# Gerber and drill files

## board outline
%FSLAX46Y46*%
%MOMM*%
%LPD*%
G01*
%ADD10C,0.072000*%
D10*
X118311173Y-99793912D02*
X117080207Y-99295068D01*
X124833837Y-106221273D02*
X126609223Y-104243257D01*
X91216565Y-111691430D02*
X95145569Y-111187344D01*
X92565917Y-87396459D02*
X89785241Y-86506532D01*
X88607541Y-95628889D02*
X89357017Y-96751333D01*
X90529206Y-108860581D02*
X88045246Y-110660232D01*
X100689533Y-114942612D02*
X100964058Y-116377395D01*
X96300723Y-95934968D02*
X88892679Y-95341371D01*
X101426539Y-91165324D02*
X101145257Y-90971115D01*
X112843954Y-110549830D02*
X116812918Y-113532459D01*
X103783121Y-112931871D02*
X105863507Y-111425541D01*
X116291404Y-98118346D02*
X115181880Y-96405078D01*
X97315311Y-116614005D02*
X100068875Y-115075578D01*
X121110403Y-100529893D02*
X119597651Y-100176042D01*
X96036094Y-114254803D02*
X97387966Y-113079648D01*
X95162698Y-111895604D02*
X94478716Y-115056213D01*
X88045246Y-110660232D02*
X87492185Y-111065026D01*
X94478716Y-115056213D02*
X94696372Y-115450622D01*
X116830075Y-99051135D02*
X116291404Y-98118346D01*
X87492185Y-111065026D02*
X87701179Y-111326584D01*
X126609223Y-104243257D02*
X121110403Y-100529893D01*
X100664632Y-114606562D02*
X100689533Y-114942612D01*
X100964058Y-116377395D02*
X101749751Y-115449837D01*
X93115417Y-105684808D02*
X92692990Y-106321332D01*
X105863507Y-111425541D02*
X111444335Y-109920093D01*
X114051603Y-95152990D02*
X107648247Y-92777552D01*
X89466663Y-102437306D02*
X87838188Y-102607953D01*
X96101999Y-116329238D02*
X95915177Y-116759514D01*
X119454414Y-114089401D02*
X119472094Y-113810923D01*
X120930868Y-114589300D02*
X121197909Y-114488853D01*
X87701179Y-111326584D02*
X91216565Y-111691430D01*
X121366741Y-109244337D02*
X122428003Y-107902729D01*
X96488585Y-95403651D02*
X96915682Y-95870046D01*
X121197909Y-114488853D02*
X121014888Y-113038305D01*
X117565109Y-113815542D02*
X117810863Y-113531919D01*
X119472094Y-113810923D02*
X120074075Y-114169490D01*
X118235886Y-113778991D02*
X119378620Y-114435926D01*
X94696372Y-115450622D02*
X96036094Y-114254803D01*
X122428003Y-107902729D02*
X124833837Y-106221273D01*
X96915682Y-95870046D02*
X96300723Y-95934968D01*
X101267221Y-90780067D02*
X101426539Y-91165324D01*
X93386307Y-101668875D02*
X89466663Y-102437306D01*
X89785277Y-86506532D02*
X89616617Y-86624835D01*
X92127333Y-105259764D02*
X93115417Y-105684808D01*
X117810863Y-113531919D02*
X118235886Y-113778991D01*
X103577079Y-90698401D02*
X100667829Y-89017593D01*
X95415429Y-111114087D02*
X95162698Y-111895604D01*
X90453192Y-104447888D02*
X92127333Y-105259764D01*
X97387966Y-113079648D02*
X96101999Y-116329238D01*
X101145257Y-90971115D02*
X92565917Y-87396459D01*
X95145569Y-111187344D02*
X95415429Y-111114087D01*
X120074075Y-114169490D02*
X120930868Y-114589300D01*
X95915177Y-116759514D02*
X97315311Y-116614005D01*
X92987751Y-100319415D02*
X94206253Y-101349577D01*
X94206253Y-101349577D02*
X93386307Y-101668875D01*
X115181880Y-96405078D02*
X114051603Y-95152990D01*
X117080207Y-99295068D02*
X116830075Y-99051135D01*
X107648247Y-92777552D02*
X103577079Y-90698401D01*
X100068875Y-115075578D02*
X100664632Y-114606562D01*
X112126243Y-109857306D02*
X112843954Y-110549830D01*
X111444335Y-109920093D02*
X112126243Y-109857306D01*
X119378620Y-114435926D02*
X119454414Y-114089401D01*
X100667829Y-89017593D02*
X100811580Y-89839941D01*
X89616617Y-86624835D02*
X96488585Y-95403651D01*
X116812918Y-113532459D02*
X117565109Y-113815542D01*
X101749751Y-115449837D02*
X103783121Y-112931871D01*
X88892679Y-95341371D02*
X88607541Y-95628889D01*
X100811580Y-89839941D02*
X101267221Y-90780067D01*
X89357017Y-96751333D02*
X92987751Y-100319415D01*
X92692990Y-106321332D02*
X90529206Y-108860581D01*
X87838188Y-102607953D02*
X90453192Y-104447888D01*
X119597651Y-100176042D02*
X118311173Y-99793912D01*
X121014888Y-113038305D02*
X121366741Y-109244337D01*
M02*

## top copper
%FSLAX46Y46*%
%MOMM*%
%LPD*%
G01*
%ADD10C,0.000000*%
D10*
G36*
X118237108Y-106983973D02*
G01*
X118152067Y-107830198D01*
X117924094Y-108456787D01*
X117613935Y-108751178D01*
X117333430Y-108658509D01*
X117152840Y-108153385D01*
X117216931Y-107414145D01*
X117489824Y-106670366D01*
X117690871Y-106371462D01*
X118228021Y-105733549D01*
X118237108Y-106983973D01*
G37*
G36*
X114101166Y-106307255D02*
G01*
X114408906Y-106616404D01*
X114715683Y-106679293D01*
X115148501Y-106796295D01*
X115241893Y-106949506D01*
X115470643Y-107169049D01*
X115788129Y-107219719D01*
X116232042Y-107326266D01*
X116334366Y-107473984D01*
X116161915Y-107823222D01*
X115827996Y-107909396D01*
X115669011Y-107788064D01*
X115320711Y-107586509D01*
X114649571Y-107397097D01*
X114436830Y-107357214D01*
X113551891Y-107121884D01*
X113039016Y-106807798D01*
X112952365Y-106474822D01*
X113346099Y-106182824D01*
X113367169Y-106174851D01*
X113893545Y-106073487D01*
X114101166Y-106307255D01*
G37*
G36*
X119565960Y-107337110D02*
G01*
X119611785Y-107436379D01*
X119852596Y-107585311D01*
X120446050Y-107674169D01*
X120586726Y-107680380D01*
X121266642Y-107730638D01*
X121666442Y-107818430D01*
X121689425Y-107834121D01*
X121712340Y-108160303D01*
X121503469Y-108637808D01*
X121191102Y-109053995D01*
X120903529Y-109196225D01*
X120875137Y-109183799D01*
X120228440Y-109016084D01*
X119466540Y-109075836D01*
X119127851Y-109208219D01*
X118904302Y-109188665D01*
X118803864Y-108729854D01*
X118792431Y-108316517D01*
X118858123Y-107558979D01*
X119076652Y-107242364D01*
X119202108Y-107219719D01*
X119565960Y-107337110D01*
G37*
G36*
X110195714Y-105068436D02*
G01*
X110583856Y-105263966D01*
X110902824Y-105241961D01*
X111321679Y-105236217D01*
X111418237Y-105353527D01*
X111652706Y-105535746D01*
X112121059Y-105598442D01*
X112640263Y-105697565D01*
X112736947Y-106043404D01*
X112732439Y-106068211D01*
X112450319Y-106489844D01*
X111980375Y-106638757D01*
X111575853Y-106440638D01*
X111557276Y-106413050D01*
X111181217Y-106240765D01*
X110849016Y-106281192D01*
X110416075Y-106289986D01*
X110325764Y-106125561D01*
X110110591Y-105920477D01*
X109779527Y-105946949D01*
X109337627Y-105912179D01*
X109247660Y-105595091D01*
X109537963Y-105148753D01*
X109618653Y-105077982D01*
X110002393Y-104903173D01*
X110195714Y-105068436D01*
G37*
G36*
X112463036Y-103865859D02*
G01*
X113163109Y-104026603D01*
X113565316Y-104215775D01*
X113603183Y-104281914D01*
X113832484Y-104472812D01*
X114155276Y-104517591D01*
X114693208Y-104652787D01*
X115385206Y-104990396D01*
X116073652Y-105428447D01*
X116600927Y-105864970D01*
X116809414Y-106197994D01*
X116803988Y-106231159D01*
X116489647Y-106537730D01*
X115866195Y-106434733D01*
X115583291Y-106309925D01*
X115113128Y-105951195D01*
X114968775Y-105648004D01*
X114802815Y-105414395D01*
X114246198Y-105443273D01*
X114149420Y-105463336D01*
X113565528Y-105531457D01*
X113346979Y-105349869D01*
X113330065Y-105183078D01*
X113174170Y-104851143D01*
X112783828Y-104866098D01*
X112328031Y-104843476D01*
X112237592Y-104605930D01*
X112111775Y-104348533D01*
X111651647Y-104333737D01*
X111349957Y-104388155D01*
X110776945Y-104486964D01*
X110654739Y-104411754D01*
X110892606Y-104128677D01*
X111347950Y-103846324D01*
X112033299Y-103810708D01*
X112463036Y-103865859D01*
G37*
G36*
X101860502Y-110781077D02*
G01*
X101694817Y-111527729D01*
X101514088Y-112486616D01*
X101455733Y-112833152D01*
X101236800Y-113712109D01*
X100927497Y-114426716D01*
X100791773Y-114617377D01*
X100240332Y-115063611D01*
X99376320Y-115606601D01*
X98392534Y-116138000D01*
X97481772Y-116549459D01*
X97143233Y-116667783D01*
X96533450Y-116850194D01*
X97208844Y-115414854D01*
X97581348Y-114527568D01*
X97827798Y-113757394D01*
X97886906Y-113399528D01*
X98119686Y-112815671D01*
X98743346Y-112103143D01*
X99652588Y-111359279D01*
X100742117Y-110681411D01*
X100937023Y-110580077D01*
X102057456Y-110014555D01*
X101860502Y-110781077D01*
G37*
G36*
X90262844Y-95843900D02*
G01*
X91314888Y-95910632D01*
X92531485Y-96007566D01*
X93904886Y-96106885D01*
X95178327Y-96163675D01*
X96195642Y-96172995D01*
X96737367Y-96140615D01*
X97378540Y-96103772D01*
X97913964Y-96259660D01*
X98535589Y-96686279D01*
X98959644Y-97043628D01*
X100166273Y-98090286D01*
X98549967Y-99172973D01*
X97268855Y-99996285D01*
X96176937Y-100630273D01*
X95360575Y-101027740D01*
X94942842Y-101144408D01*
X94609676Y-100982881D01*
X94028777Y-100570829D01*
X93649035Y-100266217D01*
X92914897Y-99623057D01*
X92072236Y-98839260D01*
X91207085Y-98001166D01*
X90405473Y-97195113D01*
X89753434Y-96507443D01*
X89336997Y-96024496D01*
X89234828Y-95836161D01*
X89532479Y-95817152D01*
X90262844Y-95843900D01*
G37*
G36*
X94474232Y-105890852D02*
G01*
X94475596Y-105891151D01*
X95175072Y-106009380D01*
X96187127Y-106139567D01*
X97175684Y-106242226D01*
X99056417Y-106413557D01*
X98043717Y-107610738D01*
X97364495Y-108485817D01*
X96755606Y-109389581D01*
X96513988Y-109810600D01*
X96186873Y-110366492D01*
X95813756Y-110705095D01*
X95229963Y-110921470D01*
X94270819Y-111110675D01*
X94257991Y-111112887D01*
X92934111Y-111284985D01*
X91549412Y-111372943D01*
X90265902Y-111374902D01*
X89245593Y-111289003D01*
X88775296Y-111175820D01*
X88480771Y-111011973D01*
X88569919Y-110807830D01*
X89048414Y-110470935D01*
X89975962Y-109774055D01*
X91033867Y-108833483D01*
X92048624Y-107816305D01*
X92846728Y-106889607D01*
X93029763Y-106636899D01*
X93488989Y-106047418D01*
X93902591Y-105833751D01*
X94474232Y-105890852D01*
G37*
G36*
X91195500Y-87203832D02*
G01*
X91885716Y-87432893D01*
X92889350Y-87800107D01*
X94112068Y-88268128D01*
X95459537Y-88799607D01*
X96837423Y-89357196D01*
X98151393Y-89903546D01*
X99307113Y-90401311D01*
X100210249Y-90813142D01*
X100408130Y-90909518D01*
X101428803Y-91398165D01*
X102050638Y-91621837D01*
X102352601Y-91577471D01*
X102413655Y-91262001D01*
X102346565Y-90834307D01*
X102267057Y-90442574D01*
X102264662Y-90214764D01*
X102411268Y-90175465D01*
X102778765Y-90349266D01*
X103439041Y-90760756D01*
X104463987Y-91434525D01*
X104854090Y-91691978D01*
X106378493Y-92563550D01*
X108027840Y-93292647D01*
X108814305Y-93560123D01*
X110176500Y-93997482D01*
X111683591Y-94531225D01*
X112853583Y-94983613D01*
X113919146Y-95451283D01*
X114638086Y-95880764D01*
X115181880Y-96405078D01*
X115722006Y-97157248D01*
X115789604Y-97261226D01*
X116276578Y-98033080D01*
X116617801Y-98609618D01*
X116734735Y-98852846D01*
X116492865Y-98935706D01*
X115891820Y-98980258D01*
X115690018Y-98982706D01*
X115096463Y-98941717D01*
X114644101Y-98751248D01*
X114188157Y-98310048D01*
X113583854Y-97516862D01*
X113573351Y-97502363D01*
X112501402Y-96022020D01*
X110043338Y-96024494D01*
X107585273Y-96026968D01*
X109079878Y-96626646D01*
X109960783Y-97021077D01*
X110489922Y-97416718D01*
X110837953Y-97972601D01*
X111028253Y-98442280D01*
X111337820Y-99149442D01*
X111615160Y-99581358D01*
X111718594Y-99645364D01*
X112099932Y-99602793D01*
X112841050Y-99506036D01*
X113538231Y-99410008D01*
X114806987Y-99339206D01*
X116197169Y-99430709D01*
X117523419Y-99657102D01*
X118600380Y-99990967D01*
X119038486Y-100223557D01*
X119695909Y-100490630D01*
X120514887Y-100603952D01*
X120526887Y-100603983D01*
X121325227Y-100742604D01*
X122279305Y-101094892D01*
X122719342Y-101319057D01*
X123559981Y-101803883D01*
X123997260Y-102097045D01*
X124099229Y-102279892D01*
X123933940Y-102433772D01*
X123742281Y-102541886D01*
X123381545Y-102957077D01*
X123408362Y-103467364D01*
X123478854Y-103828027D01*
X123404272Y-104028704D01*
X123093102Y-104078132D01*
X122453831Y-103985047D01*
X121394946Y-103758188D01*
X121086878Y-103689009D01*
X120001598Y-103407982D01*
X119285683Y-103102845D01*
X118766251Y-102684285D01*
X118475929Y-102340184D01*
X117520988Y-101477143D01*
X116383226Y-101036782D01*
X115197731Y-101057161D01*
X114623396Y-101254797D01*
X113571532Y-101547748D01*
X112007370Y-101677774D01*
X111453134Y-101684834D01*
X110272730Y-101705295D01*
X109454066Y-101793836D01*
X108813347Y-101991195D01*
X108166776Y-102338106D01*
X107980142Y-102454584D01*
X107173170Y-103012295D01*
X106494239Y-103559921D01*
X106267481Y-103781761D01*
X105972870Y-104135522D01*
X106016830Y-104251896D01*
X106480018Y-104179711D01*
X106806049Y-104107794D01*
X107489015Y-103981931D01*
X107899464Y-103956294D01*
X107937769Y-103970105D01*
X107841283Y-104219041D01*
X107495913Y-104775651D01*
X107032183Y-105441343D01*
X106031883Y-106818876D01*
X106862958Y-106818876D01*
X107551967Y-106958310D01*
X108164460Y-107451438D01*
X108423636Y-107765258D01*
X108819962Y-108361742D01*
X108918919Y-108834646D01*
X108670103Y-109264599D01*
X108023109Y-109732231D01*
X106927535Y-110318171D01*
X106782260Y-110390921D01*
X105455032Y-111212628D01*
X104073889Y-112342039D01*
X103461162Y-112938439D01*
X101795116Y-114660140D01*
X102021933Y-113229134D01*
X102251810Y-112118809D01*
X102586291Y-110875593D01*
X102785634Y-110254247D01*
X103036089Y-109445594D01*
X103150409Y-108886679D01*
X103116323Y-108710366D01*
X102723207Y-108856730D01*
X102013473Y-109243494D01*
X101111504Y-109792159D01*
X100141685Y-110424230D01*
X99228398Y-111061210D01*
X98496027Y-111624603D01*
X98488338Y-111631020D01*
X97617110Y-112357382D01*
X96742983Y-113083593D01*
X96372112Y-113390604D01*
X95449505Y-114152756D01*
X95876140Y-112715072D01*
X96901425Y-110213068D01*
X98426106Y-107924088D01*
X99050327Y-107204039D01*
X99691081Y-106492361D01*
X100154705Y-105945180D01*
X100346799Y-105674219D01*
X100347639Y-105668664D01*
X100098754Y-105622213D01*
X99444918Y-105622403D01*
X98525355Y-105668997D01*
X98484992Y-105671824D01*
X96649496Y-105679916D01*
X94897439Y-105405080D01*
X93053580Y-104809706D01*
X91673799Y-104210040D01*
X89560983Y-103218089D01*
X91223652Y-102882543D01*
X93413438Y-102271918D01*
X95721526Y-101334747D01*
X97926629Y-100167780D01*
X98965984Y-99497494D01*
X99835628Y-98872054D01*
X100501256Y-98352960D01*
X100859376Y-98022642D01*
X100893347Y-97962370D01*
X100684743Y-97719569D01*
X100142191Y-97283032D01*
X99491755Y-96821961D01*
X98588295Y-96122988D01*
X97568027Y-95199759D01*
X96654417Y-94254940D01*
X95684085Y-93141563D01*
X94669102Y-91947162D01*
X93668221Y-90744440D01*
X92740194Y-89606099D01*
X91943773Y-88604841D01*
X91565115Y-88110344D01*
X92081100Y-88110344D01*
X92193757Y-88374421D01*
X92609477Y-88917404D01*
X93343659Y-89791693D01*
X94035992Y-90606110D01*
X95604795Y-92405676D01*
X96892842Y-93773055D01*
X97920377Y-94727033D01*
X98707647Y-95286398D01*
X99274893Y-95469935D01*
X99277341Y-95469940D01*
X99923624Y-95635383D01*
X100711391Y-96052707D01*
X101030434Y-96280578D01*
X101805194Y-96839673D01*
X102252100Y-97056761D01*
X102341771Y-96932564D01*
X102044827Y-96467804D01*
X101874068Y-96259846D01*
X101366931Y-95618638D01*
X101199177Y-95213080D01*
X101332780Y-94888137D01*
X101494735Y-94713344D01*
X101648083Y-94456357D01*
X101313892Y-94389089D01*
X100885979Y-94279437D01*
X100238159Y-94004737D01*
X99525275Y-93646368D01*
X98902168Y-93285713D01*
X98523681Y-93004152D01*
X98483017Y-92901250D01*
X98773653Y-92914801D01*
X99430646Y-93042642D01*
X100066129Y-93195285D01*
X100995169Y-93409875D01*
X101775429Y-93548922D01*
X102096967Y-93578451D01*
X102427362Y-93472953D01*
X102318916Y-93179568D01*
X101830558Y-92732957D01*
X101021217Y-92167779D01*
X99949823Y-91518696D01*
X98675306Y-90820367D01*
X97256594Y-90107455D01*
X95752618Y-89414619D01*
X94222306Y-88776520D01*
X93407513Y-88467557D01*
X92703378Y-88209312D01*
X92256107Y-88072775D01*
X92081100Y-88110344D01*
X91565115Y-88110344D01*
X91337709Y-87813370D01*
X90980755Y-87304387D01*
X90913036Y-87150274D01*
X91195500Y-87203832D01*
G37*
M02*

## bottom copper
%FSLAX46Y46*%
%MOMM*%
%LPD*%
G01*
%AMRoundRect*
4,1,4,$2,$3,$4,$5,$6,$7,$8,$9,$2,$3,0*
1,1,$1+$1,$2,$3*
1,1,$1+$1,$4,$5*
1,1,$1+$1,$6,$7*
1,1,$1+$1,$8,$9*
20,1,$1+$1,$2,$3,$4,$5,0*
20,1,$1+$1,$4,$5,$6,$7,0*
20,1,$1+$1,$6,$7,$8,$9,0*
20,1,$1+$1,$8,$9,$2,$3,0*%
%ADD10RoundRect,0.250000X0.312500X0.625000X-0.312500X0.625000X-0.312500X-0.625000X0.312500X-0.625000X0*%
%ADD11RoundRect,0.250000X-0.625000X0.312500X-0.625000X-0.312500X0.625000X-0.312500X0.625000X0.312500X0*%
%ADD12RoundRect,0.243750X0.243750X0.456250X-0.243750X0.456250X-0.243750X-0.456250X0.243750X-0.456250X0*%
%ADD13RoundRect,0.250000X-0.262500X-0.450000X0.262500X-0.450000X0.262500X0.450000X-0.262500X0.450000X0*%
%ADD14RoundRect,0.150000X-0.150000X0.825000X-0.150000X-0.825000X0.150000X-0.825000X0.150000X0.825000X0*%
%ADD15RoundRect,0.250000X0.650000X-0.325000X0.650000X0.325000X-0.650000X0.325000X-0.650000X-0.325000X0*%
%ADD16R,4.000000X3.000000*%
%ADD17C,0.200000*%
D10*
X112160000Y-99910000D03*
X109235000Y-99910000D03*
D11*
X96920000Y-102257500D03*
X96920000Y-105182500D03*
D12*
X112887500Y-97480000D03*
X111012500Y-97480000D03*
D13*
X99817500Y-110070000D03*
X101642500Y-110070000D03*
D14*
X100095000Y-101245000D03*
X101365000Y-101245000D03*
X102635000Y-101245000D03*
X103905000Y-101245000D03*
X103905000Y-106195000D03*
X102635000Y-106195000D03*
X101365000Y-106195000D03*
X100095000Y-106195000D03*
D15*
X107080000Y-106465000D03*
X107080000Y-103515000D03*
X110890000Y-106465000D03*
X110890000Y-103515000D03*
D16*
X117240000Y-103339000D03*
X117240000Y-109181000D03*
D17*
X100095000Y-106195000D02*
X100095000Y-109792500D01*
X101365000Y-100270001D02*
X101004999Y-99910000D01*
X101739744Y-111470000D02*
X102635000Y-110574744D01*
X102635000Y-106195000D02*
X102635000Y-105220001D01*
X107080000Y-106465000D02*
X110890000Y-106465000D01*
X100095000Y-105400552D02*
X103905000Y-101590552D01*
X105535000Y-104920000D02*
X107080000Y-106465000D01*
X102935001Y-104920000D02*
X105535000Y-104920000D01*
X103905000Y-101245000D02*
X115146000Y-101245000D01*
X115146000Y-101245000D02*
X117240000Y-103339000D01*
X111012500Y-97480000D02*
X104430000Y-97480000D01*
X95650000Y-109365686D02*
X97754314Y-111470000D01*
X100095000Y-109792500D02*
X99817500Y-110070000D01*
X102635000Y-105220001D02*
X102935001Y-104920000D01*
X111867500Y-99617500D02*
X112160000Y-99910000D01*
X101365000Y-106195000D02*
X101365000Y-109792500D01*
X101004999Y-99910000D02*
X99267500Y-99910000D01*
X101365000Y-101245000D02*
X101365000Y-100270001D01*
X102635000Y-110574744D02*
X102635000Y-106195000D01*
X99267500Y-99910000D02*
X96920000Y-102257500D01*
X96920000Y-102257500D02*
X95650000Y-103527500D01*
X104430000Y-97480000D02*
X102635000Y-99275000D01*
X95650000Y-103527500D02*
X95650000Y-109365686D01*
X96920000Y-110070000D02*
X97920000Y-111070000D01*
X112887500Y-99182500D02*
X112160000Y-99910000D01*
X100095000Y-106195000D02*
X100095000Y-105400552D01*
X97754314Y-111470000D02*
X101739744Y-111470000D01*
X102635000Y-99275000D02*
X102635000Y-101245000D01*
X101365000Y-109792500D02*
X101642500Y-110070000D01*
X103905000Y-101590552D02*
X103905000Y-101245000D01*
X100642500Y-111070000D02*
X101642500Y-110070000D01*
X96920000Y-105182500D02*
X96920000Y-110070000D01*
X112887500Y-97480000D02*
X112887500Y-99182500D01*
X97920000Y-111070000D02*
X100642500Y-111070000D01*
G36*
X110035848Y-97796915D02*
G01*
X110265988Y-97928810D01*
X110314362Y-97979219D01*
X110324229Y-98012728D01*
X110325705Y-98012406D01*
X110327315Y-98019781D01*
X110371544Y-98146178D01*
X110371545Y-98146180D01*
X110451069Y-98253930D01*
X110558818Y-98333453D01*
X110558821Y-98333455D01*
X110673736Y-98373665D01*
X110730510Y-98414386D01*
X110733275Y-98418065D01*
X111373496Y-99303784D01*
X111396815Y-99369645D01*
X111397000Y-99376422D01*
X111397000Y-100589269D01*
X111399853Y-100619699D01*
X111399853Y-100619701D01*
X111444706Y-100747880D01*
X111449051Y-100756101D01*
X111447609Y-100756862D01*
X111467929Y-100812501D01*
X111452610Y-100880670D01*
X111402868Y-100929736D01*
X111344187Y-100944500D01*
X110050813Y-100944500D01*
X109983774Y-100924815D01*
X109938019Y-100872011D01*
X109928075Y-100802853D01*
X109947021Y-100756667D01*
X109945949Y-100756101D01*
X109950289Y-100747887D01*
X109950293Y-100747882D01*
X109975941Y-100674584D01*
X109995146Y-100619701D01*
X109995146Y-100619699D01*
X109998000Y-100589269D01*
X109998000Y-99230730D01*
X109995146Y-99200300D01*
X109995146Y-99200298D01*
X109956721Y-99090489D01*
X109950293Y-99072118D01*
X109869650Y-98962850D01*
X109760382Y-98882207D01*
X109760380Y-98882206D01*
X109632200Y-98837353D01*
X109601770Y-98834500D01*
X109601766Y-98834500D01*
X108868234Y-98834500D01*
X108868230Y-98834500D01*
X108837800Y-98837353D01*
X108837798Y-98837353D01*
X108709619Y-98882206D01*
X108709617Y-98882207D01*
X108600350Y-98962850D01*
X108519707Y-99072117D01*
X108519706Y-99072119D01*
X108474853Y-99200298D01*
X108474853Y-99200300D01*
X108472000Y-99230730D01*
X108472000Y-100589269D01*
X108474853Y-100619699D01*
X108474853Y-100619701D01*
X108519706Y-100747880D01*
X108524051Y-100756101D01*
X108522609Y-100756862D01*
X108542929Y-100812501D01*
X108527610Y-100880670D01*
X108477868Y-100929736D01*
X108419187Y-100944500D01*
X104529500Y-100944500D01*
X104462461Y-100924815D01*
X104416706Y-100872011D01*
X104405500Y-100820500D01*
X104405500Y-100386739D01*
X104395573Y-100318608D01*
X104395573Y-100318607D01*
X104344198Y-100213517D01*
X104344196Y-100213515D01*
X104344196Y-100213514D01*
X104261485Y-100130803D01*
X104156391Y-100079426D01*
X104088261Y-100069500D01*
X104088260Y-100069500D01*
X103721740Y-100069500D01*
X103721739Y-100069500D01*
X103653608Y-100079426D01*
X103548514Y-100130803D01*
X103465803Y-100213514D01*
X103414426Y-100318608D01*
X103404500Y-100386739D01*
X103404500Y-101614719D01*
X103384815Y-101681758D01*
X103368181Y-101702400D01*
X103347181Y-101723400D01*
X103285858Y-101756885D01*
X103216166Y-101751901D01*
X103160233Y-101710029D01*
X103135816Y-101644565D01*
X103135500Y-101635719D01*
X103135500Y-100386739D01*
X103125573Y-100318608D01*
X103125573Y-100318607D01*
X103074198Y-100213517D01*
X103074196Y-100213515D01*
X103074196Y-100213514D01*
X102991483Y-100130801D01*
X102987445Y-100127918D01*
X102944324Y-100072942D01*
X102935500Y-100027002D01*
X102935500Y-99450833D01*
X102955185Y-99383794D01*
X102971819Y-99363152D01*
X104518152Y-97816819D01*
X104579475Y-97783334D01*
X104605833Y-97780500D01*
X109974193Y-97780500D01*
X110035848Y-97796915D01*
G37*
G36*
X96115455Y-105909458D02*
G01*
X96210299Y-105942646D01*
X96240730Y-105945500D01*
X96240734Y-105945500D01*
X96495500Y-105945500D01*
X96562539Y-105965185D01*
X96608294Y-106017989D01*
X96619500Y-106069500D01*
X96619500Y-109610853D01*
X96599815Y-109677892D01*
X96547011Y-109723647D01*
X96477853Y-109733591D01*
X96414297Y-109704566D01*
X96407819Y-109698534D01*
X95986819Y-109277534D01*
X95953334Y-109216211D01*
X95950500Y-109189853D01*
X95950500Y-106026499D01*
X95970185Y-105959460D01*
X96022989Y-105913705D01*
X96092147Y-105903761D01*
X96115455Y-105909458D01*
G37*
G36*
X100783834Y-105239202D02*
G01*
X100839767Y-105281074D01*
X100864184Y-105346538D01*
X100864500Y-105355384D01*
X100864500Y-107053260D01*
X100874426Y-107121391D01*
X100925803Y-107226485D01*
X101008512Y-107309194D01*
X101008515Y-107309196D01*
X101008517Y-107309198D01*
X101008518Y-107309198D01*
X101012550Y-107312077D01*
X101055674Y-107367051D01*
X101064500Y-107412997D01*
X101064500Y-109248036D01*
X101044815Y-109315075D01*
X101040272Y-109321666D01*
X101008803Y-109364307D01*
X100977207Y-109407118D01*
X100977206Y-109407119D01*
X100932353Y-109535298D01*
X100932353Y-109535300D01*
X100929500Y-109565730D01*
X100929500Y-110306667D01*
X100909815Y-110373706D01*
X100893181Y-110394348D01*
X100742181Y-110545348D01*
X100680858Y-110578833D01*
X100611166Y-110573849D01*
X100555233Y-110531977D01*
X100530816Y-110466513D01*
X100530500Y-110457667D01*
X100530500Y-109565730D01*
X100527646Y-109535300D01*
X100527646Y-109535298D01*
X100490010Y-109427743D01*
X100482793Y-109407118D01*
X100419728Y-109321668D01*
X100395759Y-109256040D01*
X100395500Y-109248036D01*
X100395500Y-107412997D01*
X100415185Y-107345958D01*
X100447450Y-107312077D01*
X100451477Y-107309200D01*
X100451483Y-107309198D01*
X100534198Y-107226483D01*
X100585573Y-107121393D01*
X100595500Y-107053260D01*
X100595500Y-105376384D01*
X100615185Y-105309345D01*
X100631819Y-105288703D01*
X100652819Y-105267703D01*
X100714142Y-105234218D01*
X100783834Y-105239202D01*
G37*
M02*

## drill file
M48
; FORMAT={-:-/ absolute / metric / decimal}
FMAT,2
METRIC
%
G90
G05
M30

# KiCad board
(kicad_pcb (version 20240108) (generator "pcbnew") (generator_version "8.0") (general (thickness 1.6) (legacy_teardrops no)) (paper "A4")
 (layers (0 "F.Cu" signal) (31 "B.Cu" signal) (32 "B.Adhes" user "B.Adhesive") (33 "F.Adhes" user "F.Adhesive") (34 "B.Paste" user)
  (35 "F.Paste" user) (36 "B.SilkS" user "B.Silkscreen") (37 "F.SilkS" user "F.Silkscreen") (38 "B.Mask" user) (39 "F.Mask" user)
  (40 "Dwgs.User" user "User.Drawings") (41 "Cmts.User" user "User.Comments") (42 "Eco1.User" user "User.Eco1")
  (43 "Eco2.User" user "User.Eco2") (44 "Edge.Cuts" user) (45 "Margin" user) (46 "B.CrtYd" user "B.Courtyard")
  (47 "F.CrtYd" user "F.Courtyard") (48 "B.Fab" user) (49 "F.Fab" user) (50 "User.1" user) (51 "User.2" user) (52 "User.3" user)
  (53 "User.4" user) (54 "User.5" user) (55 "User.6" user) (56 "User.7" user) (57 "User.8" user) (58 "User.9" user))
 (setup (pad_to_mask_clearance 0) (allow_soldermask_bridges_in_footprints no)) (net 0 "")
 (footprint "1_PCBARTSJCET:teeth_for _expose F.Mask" (layer "F.Cu") (at 115.888129 157.599293)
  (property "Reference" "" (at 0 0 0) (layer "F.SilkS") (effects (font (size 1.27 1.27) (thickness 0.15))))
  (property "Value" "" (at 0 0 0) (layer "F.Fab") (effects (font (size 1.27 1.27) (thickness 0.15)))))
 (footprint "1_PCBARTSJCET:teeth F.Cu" (layer "F.Cu") (at 115.788129 157.479293)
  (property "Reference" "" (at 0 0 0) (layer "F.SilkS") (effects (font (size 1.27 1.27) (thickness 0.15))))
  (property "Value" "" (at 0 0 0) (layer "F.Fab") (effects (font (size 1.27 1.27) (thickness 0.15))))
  (fp_poly
   (pts (xy 2.448979 -50.49532) (xy 2.363938 -49.649095) (xy 2.135965 -49.022506) (xy 1.825806 -48.728115) (xy 1.545301 -48.820784)
    (xy 1.364711 -49.325908) (xy 1.428802 -50.065148) (xy 1.701695 -50.808927) (xy 1.902742 -51.107831) (xy 2.439892 -51.745744))
   (stroke (width 0) (type solid)) (fill solid) (layer "F.Cu"))
  (fp_poly
   (pts (xy -1.686963 -51.172038) (xy -1.379223 -50.862889) (xy -1.072446 -50.8) (xy -0.639628 -50.682998) (xy -0.546236 -50.529787)
    (xy -0.317486 -50.310244) (xy 0 -50.259574) (xy 0.443913 -50.153027) (xy 0.546237 -50.005309) (xy 0.373786 -49.656071)
    (xy 0.039867 -49.569897) (xy -0.119118 -49.691229) (xy -0.467418 -49.892784) (xy -1.138558 -50.082196) (xy -1.351299 -50.122079)
    (xy -2.236238 -50.357409) (xy -2.749113 -50.671495) (xy -2.835764 -51.004471) (xy -2.44203 -51.296469) (xy -2.42096 -51.304442)
    (xy -1.894584 -51.405806))
   (stroke (width 0) (type solid)) (fill solid) (layer "F.Cu"))
  (fp_poly
   (pts (xy 3.777831 -50.142183) (xy 3.823656 -50.042914) (xy 4.064467 -49.893982) (xy 4.657921 -49.805124) (xy 4.798597 -49.798913)
    (xy 5.478513 -49.748655) (xy 5.878313 -49.660863) (xy 5.901296 -49.645172) (xy 5.924211 -49.31899) (xy 5.71534 -48.841485)
    (xy 5.402973 -48.425298) (xy 5.1154 -48.283068) (xy 5.087008 -48.295494) (xy 4.440311 -48.463209) (xy 3.678411 -48.403457)
    (xy 3.339722 -48.271074) (xy 3.116173 -48.290628) (xy 3.015735 -48.749439) (xy 3.004302 -49.162776) (xy 3.069994 -49.920314)
    (xy 3.288523 -50.236929) (xy 3.413979 -50.259574))
   (stroke (width 0) (type solid)) (fill solid) (layer "F.Cu"))
  (fp_poly
   (pts (xy -5.592415 -52.410857) (xy -5.204273 -52.215327) (xy -4.885305 -52.237332) (xy -4.46645 -52.243076) (xy -4.369892 -52.125766)
    (xy -4.135423 -51.943547) (xy -3.66707 -51.880851) (xy -3.147866 -51.781728) (xy -3.051182 -51.435889) (xy -3.05569 -51.411082)
    (xy -3.33781 -50.989449) (xy -3.807754 -50.840536) (xy -4.212276 -51.038655) (xy -4.230853 -51.066243) (xy -4.606912 -51.238528)
    (xy -4.939113 -51.198101) (xy -5.372054 -51.189307) (xy -5.462365 -51.353732) (xy -5.677538 -51.558816) (xy -6.008602 -51.532344)
    (xy -6.450502 -51.567114) (xy -6.540469 -51.884202) (xy -6.250166 -52.33054) (xy -6.169476 -52.401311) (xy -5.785736 -52.57612))
   (stroke (width 0) (type solid)) (fill solid) (layer "F.Cu"))
  (fp_poly
   (pts (xy -3.325093 -53.613434) (xy -2.62502 -53.45269) (xy -2.222813 -53.263518) (xy -2.184946 -53.197379) (xy -1.955645 -53.006481)
    (xy -1.632853 -52.961702) (xy -1.094921 -52.826506) (xy -0.402923 -52.488897) (xy 0.285523 -52.050846) (xy 0.812798 -51.614323)
    (xy 1.021285 -51.281299) (xy 1.015859 -51.248134) (xy 0.701518 -50.941563) (xy 0.078066 -51.04456) (xy -0.204838 -51.169368)
    (xy -0.675001 -51.528098) (xy -0.819354 -51.831289) (xy -0.985314 -52.064898) (xy -1.541931 -52.03602) (xy -1.638709 -52.015957)
    (xy -2.222601 -51.947836) (xy -2.44115 -52.129424) (xy -2.458064 -52.296215) (xy -2.613959 -52.62815) (xy -3.004301 -52.613195)
    (xy -3.460098 -52.635817) (xy -3.550537 -52.873363) (xy -3.676354 -53.13076) (xy -4.136482 -53.145556) (xy -4.438172 -53.091138)
    (xy -5.011184 -52.992329) (xy -5.13339 -53.067539) (xy -4.895523 -53.350616) (xy -4.440179 -53.632969) (xy -3.75483 -53.668585))
   (stroke (width 0) (type solid)) (fill solid) (layer "F.Cu")))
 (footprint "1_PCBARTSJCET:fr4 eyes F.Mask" (layer "F.Cu") (at 121.93 155.57)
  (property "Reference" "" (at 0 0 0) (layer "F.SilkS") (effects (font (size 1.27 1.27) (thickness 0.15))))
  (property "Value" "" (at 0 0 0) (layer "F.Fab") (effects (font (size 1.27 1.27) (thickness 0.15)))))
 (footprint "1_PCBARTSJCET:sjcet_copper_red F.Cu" (layer "F.Cu") (at 114.822907 158.699727)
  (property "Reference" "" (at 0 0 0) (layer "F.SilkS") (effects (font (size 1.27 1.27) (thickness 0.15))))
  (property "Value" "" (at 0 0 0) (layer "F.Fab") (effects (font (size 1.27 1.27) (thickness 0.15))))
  (fp_poly
   (pts (xy -12.962405 -47.91865) (xy -13.12809 -47.171998) (xy -13.308819 -46.213111) (xy -13.367174 -45.866575) (xy -13.586107 -44.987618)
    (xy -13.89541 -44.273011) (xy -14.031134 -44.08235) (xy -14.582575 -43.636116) (xy -15.446587 -43.093126) (xy -16.430373 -42.561727)
    (xy -17.341135 -42.150268) (xy -17.679674 -42.031944) (xy -18.289457 -41.849533) (xy -17.614063 -43.284873) (xy -17.241559 -44.172159)
    (xy -16.995109 -44.942333) (xy -16.936001 -45.300199) (xy -16.703221 -45.884056) (xy -16.079561 -46.596584) (xy -15.170319 -47.340448)
    (xy -14.08079 -48.018316) (xy -13.885884 -48.11965) (xy -12.765451 -48.685172))
   (stroke (width 0) (type solid)) (fill solid) (layer "F.Cu"))
  (fp_poly
   (pts (xy -24.560063 -62.855827) (xy -23.508019 -62.789095) (xy -22.291422 -62.692161) (xy -20.918021 -62.592842)
    (xy -19.64458 -62.536052) (xy -18.627265 -62.526732) (xy -18.08554 -62.559112) (xy -17.444367 -62.595955) (xy -16.908943 -62.440067)
    (xy -16.287318 -62.013448) (xy -15.863263 -61.656099) (xy -14.656634 -60.609441) (xy -16.27294 -59.526754) (xy -17.554052 -58.703442)
    (xy -18.64597 -58.069454) (xy -19.462332 -57.671987) (xy -19.880065 -57.555319) (xy -20.213231 -57.716846) (xy -20.79413 -58.128898)
    (xy -21.173872 -58.43351) (xy -21.90801 -59.07667) (xy -22.750671 -59.860467) (xy -23.615822 -60.698561) (xy -24.417434 -61.504614)
    (xy -25.069473 -62.192284) (xy -25.48591 -62.675231) (xy -25.588079 -62.863566) (xy -25.290428 -62.882575))
   (stroke (width 0) (type solid)) (fill solid) (layer "F.Cu"))
  (fp_poly
   (pts (xy -20.348675 -52.808875) (xy -20.347311 -52.808576) (xy -19.647835 -52.690347) (xy -18.63578 -52.56016) (xy -17.647223 -52.457501)
    (xy -15.76649 -52.28617) (xy -16.77919 -51.088989) (xy -17.458412 -50.21391) (xy -18.067301 -49.310146) (xy -18.308919 -48.889127)
    (xy -18.636034 -48.333235) (xy -19.009151 -47.994632) (xy -19.592944 -47.778257) (xy -20.552088 -47.589052) (xy -20.564916 -47.58684)
    (xy -21.888796 -47.414742) (xy -23.273495 -47.326784) (xy -24.557005 -47.324825) (xy -25.577314 -47.410724) (xy -26.047611 -47.523907)
    (xy -26.342136 -47.687754) (xy -26.252988 -47.891897) (xy -25.774493 -48.228792) (xy -24.846945 -48.925672) (xy -23.78904 -49.866244)
    (xy -22.774283 -50.883422) (xy -21.976179 -51.81012) (xy -21.793144 -52.062828) (xy -21.333918 -52.652309) (xy -20.920316 -52.865976))
   (stroke (width 0) (type solid)) (fill solid) (layer "F.Cu"))
  (fp_poly
   (pts (xy -23.627407 -71.495895) (xy -22.937191 -71.266834) (xy -21.933557 -70.89962) (xy -20.710839 -70.431599) (xy -19.36337 -69.90012)
    (xy -17.985484 -69.342531) (xy -16.671514 -68.796181) (xy -15.515794 -68.298416) (xy -14.612658 -67.886585) (xy -14.414777 -67.790209)
    (xy -13.394104 -67.301562) (xy -12.772269 -67.07789) (xy -12.470306 -67.122256) (xy -12.409252 -67.437726) (xy -12.476342 -67.86542)
    (xy -12.55585 -68.257153) (xy -12.558245 -68.484963) (xy -12.411639 -68.524262) (xy -12.044142 -68.350461) (xy -11.383866 -67.938971)
    (xy -10.35892 -67.265202) (xy -9.968817 -67.007749) (xy -8.444414 -66.136177) (xy -6.795067 -65.40708) (xy -6.008602 -65.139604)
    (xy -4.646407 -64.702245) (xy -3.139316 -64.168502) (xy -1.969324 -63.716114) (xy -0.903761 -63.248444) (xy -0.184821 -62.818963)
    (xy 0.358973 -62.294649) (xy 0.899099 -61.542479) (xy 0.966697 -61.438501) (xy 1.453671 -60.666647) (xy 1.794894 -60.090109)
    (xy 1.911828 -59.846881) (xy 1.669958 -59.764021) (xy 1.068913 -59.719469) (xy 0.867111 -59.717021) (xy 0.273556 -59.75801)
    (xy -0.178806 -59.948479) (xy -0.63475 -60.389679) (xy -1.239053 -61.182865) (xy -1.249556 -61.197364) (xy -2.321505 -62.677707)
    (xy -4.779569 -62.675233) (xy -7.237634 -62.672759) (xy -5.743029 -62.073081) (xy -4.862124 -61.67865) (xy -4.332985 -61.283009)
    (xy -3.984954 -60.727126) (xy -3.794654 -60.257447) (xy -3.485087 -59.550285) (xy -3.207747 -59.118369) (xy -3.104313 -59.054363)
    (xy -2.722975 -59.096934) (xy -1.981857 -59.193691) (xy -1.284676 -59.289719) (xy -0.01592 -59.360521) (xy 1.374262 -59.269018)
    (xy 2.700512 -59.042625) (xy 3.777473 -58.70876) (xy 4.215579 -58.47617) (xy 4.873002 -58.209097) (xy 5.69198 -58.095775)
    (xy 5.70398 -58.095744) (xy 6.50232 -57.957123) (xy 7.456398 -57.604835) (xy 7.896435 -57.38067) (xy 8.737074 -56.895844)
    (xy 9.174353 -56.602682) (xy 9.276322 -56.419835) (xy 9.111033 -56.265955) (xy 8.919374 -56.157841) (xy 8.558638 -55.74265)
    (xy 8.585455 -55.232363) (xy 8.655947 -54.8717) (xy 8.581365 -54.671023) (xy 8.270195 -54.621595) (xy 7.630924 -54.71468)
    (xy 6.572039 -54.941539) (xy 6.263971 -55.010718) (xy 5.178691 -55.291745) (xy 4.462776 -55.596882) (xy 3.943344 -56.015442)
    (xy 3.653022 -56.359543) (xy 2.698081 -57.222584) (xy 1.560319 -57.662945) (xy 0.374824 -57.642566) (xy -0.199511 -57.44493)
    (xy -1.251375 -57.151979) (xy -2.815537 -57.021953) (xy -3.369773 -57.014893) (xy -4.550177 -56.994432) (xy -5.368841 -56.905891)
    (xy -6.00956 -56.708532) (xy -6.656131 -56.361621) (xy -6.842765 -56.245143) (xy -7.649737 -55.687432) (xy -8.328668 -55.139806)
    (xy -8.555426 -54.917966) (xy -8.850037 -54.564205) (xy -8.806077 -54.447831) (xy -8.342889 -54.520016) (xy -8.016858 -54.591933)
    (xy -7.333892 -54.717796) (xy -6.923443 -54.743433) (xy -6.885138 -54.729622) (xy -6.981624 -54.480686) (xy -7.326994 -53.924076)
    (xy -7.790724 -53.258384) (xy -8.791024 -51.880851) (xy -7.959949 -51.880851) (xy -7.27094 -51.741417) (xy -6.658447 -51.248289)
    (xy -6.399271 -50.934469) (xy -6.002945 -50.337985) (xy -5.903988 -49.865081) (xy -6.152804 -49.435128) (xy -6.799798 -48.967496)
    (xy -7.895372 -48.381556) (xy -8.040647 -48.308806) (xy -9.367875 -47.487099) (xy -10.749018 -46.357688) (xy -11.361745 -45.761288)
    (xy -13.027791 -44.039587) (xy -12.800974 -45.470593) (xy -12.571097 -46.580918) (xy -12.236616 -47.824134) (xy -12.037273 -48.44548)
    (xy -11.786818 -49.254133) (xy -11.672498 -49.813048) (xy -11.706584 -49.989361) (xy -12.0997 -49.842997) (xy -12.809434 -49.456233)
    (xy -13.711403 -48.907568) (xy -14.681222 -48.275497) (xy -15.594509 -47.638517) (xy -16.32688 -47.075124) (xy -16.334569 -47.068707)
    (xy -17.205797 -46.342345) (xy -18.079924 -45.616134) (xy -18.450795 -45.309123) (xy -19.373402 -44.546971) (xy -18.946767 -45.984655)
    (xy -17.921482 -48.486659) (xy -16.396801 -50.775639) (xy -15.77258 -51.495688) (xy -15.131826 -52.207366) (xy -14.668202 -52.754547)
    (xy -14.476108 -53.025508) (xy -14.475268 -53.031063) (xy -14.724153 -53.077514) (xy -15.377989 -53.077324) (xy -16.297552 -53.03073)
    (xy -16.337915 -53.027903) (xy -18.173411 -53.019811) (xy -19.925468 -53.294647) (xy -21.769327 -53.890021) (xy -23.149108 -54.489687)
    (xy -25.261924 -55.481638) (xy -23.599255 -55.817184) (xy -21.409469 -56.427809) (xy -19.101381 -57.36498) (xy -16.896278 -58.531947)
    (xy -15.856923 -59.202233) (xy -14.987279 -59.827673) (xy -14.321651 -60.346767) (xy -13.963531 -60.677085) (xy -13.92956 -60.737357)
    (xy -14.138164 -60.980158) (xy -14.680716 -61.416695) (xy -15.331152 -61.877766) (xy -16.234612 -62.576739) (xy -17.25488 -63.499968)
    (xy -18.16849 -64.444787) (xy -19.138822 -65.558164) (xy -20.153805 -66.752565) (xy -21.154686 -67.955287) (xy -22.082713 -69.093628)
    (xy -22.879134 -70.094886) (xy -23.257792 -70.589383) (xy -22.741807 -70.589383) (xy -22.62915 -70.325306) (xy -22.21343 -69.782323)
    (xy -21.479248 -68.908034) (xy -20.786915 -68.093617) (xy -19.218112 -66.294051) (xy -17.930065 -64.926672) (xy -16.90253 -63.972694)
    (xy -16.11526 -63.413329) (xy -15.548014 -63.229792) (xy -15.545566 -63.229787) (xy -14.899283 -63.064344) (xy -14.111516 -62.64702)
    (xy -13.792473 -62.419149) (xy -13.017713 -61.860054) (xy -12.570807 -61.642966) (xy -12.481136 -61.767163) (xy -12.77808 -62.231923)
    (xy -12.948839 -62.439881) (xy -13.455976 -63.081089) (xy -13.62373 -63.486647) (xy -13.490127 -63.81159) (xy -13.328172 -63.986383)
    (xy -13.174824 -64.24337) (xy -13.509015 -64.310638) (xy -13.936928 -64.42029) (xy -14.584748 -64.69499) (xy -15.297632 -65.053359)
    (xy -15.920739 -65.414014) (xy -16.299226 -65.695575) (xy -16.33989 -65.798477) (xy -16.049254 -65.784926) (xy -15.392261 -65.657085)
    (xy -14.756778 -65.504442) (xy -13.827738 -65.289852) (xy -13.047478 -65.150805) (xy -12.72594 -65.121276) (xy -12.395545 -65.226774)
    (xy -12.503991 -65.520159) (xy -12.992349 -65.96677) (xy -13.80169 -66.531948) (xy -14.873084 -67.181031) (xy -16.147601 -67.87936)
    (xy -17.566313 -68.592272) (xy -19.070289 -69.285108) (xy -20.600601 -69.923207) (xy -21.415394 -70.23217) (xy -22.119529 -70.490415)
    (xy -22.5668 -70.626952) (xy -22.741807 -70.589383) (xy -23.257792 -70.589383) (xy -23.485198 -70.886357) (xy -23.842152 -71.39534)
    (xy -23.909871 -71.549453))
   (stroke (width 0) (type solid)) (fill solid) (layer "F.Cu")))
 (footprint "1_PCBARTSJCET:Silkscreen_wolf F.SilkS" (layer "F.Cu") (at 107.93 104.28)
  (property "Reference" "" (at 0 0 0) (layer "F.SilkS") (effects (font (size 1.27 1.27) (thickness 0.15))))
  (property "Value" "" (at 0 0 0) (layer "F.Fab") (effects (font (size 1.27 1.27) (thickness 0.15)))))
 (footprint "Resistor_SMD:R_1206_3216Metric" (layer "B.Cu") (at 110.6975 99.91 180)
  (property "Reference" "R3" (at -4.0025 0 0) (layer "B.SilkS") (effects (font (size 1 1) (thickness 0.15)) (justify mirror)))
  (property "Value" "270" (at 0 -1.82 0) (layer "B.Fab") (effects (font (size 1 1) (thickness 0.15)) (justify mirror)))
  (pad "1" smd roundrect (at -1.4625 0 180) (size 1.125 1.75) (layers "B.Cu" "B.Paste" "B.Mask") (roundrect_rratio 0.222222))
  (pad "2" smd roundrect (at 1.4625 0 180) (size 1.125 1.75) (layers "B.Cu" "B.Paste" "B.Mask") (roundrect_rratio 0.222222)))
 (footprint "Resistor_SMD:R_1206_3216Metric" (layer "B.Cu") (at 96.92 103.72 -90)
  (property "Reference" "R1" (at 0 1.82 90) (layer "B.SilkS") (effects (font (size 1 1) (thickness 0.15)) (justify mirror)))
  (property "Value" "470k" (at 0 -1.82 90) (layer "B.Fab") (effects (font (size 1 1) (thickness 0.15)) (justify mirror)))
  (pad "1" smd roundrect (at -1.4625 0 270) (size 1.125 1.75) (layers "B.Cu" "B.Paste" "B.Mask") (roundrect_rratio 0.222222))
  (pad "2" smd roundrect (at 1.4625 0 270) (size 1.125 1.75) (layers "B.Cu" "B.Paste" "B.Mask") (roundrect_rratio 0.222222)))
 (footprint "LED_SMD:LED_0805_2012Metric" (layer "B.Cu") (at 111.95 97.48 180)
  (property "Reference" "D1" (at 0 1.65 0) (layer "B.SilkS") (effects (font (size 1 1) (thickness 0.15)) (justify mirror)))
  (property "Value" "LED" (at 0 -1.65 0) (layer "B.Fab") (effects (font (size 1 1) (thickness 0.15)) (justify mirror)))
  (pad "1" smd roundrect (at -0.9375 0 180) (size 0.975 1.4) (layers "B.Cu" "B.Paste" "B.Mask") (roundrect_rratio 0.25))
  (pad "2" smd roundrect (at 0.9375 0 180) (size 0.975 1.4) (layers "B.Cu" "B.Paste" "B.Mask") (roundrect_rratio 0.25)))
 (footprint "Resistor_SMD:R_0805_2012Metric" (layer "B.Cu") (at 100.73 110.07)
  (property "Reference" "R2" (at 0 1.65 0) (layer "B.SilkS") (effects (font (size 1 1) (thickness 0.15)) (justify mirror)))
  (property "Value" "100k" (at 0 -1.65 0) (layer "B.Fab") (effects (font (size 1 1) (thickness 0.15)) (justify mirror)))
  (pad "1" smd roundrect (at -0.9125 0) (size 1.025 1.4) (layers "B.Cu" "B.Paste" "B.Mask") (roundrect_rratio 0.243902))
  (pad "2" smd roundrect (at 0.9125 0) (size 1.025 1.4) (layers "B.Cu" "B.Paste" "B.Mask") (roundrect_rratio 0.243902)))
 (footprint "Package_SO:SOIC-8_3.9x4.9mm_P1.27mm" (layer "B.Cu") (at 102 103.72 -90)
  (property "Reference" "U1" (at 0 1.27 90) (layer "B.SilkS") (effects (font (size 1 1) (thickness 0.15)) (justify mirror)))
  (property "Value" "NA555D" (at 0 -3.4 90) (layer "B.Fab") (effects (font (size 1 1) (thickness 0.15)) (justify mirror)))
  (pad "1" smd roundrect (at -2.475 1.905 270) (size 1.95 0.6) (layers "B.Cu" "B.Paste" "B.Mask") (roundrect_rratio 0.25))
  (pad "2" smd roundrect (at -2.475 0.635 270) (size 1.95 0.6) (layers "B.Cu" "B.Paste" "B.Mask") (roundrect_rratio 0.25))
  (pad "3" smd roundrect (at -2.475 -0.635 270) (size 1.95 0.6) (layers "B.Cu" "B.Paste" "B.Mask") (roundrect_rratio 0.25))
  (pad "4" smd roundrect (at -2.475 -1.905 270) (size 1.95 0.6) (layers "B.Cu" "B.Paste" "B.Mask") (roundrect_rratio 0.25))
  (pad "5" smd roundrect (at 2.475 -1.905 270) (size 1.95 0.6) (layers "B.Cu" "B.Paste" "B.Mask") (roundrect_rratio 0.25))
  (pad "6" smd roundrect (at 2.475 -0.635 270) (size 1.95 0.6) (layers "B.Cu" "B.Paste" "B.Mask") (roundrect_rratio 0.25))
  (pad "7" smd roundrect (at 2.475 0.635 270) (size 1.95 0.6) (layers "B.Cu" "B.Paste" "B.Mask") (roundrect_rratio 0.25))
  (pad "8" smd roundrect (at 2.475 1.905 270) (size 1.95 0.6) (layers "B.Cu" "B.Paste" "B.Mask") (roundrect_rratio 0.25)))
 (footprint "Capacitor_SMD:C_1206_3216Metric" (layer "B.Cu") (at 107.08 104.99 90)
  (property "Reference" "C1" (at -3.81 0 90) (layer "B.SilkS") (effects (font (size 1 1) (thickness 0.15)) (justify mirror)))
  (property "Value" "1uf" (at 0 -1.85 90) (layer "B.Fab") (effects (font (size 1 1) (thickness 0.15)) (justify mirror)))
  (pad "1" smd roundrect (at -1.475 0 90) (size 1.15 1.8) (layers "B.Cu" "B.Paste" "B.Mask") (roundrect_rratio 0.217391))
  (pad "2" smd roundrect (at 1.475 0 90) (size 1.15 1.8) (layers "B.Cu" "B.Paste" "B.Mask") (roundrect_rratio 0.217391)))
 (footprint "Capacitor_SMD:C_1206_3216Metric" (layer "B.Cu") (at 110.89 104.99 90)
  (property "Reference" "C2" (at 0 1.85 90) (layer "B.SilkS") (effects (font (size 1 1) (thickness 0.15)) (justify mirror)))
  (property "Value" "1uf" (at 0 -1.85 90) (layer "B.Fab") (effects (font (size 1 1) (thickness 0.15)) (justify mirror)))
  (pad "1" smd roundrect (at -1.475 0 90) (size 1.15 1.8) (layers "B.Cu" "B.Paste" "B.Mask") (roundrect_rratio 0.217391))
  (pad "2" smd roundrect (at 1.475 0 90) (size 1.15 1.8) (layers "B.Cu" "B.Paste" "B.Mask") (roundrect_rratio 0.217391)))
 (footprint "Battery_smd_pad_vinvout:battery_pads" (layer "B.Cu") (at 109.62 105.625 -90)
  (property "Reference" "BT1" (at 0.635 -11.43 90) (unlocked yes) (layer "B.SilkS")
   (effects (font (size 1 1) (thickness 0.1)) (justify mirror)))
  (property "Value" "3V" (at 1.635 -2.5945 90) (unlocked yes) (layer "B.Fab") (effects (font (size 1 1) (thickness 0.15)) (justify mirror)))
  (pad "1" smd rect (at -2.286 -7.62 270) (size 3 4) (layers "B.Cu" "B.Paste" "B.Mask"))
  (pad "2" smd rect (at 3.556 -7.62 270) (size 3 4) (layers "B.Cu" "B.Paste" "B.Mask")))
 (gr_line (start 118.311173 99.793912) (end 117.080207 99.295068) (stroke (width 0.072) (type default)) (layer "Edge.Cuts"))
 (gr_line (start 124.833837 106.221273) (end 126.609223 104.243257) (stroke (width 0.072) (type default)) (layer "Edge.Cuts"))
 (gr_line (start 91.216565 111.69143) (end 95.145569 111.187344) (stroke (width 0.072) (type default)) (layer "Edge.Cuts"))
 (gr_line (start 92.565917 87.396459) (end 89.785241 86.506532) (stroke (width 0.072) (type default)) (layer "Edge.Cuts"))
 (gr_line (start 88.607541 95.628889) (end 89.357017 96.751333) (stroke (width 0.072) (type default)) (layer "Edge.Cuts"))
 (gr_line (start 90.529206 108.860581) (end 88.045246 110.660232) (stroke (width 0.072) (type default)) (layer "Edge.Cuts"))
 (gr_line (start 100.689533 114.942612) (end 100.964058 116.377395) (stroke (width 0.072) (type default)) (layer "Edge.Cuts"))
 (gr_line (start 96.300723 95.934968) (end 88.892679 95.341371) (stroke (width 0.072) (type default)) (layer "Edge.Cuts"))
 (gr_line (start 101.426539 91.165324) (end 101.145257 90.971115) (stroke (width 0.072) (type default)) (layer "Edge.Cuts"))
 (gr_line (start 112.843954 110.54983) (end 116.812918 113.532459) (stroke (width 0.072) (type default)) (layer "Edge.Cuts"))
 (gr_line (start 103.783121 112.931871) (end 105.863507 111.425541) (stroke (width 0.072) (type default)) (layer "Edge.Cuts"))
 (gr_line (start 116.291404 98.118346) (end 115.18188 96.405078) (stroke (width 0.072) (type default)) (layer "Edge.Cuts"))
 (gr_line (start 97.315311 116.614005) (end 100.068875 115.075578) (stroke (width 0.072) (type default)) (layer "Edge.Cuts"))
 (gr_line (start 121.110403 100.529893) (end 119.597651 100.176042) (stroke (width 0.072) (type default)) (layer "Edge.Cuts"))
 (gr_line (start 96.036094 114.254803) (end 97.387966 113.079648) (stroke (width 0.072) (type default)) (layer "Edge.Cuts"))
 (gr_line (start 95.162698 111.895604) (end 94.478716 115.056213) (stroke (width 0.072) (type default)) (layer "Edge.Cuts"))
 (gr_line (start 88.045246 110.660232) (end 87.492185 111.065026) (stroke (width 0.072) (type default)) (layer "Edge.Cuts"))
 (gr_line (start 94.478716 115.056213) (end 94.696372 115.450622) (stroke (width 0.072) (type default)) (layer "Edge.Cuts"))
 (gr_line (start 116.830075 99.051135) (end 116.291404 98.118346) (stroke (width 0.072) (type default)) (layer "Edge.Cuts"))
 (gr_line (start 87.492185 111.065026) (end 87.701179 111.326584) (stroke (width 0.072) (type default)) (layer "Edge.Cuts"))
 (gr_line (start 126.609223 104.243257) (end 121.110403 100.529893) (stroke (width 0.072) (type default)) (layer "Edge.Cuts"))
 (gr_line (start 100.664632 114.606562) (end 100.689533 114.942612) (stroke (width 0.072) (type default)) (layer "Edge.Cuts"))
 (gr_line (start 100.964058 116.377395) (end 101.749751 115.449837) (stroke (width 0.072) (type default)) (layer "Edge.Cuts"))
 (gr_line (start 93.115417 105.684808) (end 92.69299 106.321332) (stroke (width 0.072) (type default)) (layer "Edge.Cuts"))
 (gr_line (start 105.863507 111.425541) (end 111.444335 109.920093) (stroke (width 0.072) (type default)) (layer "Edge.Cuts"))
 (gr_line (start 114.051603 95.15299) (end 107.648247 92.777552) (stroke (width 0.072) (type default)) (layer "Edge.Cuts"))
 (gr_line (start 89.466663 102.437306) (end 87.838188 102.607953) (stroke (width 0.072) (type default)) (layer "Edge.Cuts"))
 (gr_line (start 96.101999 116.329238) (end 95.915177 116.759514) (stroke (width 0.072) (type default)) (layer "Edge.Cuts"))
 (gr_line (start 119.454414 114.089401) (end 119.472094 113.810923) (stroke (width 0.072) (type default)) (layer "Edge.Cuts"))
 (gr_line (start 120.930868 114.5893) (end 121.197909 114.488853) (stroke (width 0.072) (type default)) (layer "Edge.Cuts"))
 (gr_line (start 87.701179 111.326584) (end 91.216565 111.69143) (stroke (width 0.072) (type default)) (layer "Edge.Cuts"))
 (gr_line (start 121.366741 109.244337) (end 122.428003 107.902729) (stroke (width 0.072) (type default)) (layer "Edge.Cuts"))
 (gr_line (start 96.488585 95.403651) (end 96.915682 95.870046) (stroke (width 0.072) (type default)) (layer "Edge.Cuts"))
 (gr_line (start 121.197909 114.488853) (end 121.014888 113.038305) (stroke (width 0.072) (type default)) (layer "Edge.Cuts"))
 (gr_line (start 117.565109 113.815542) (end 117.810863 113.531919) (stroke (width 0.072) (type default)) (layer "Edge.Cuts"))
 (gr_line (start 119.472094 113.810923) (end 120.074075 114.16949) (stroke (width 0.072) (type default)) (layer "Edge.Cuts"))
 (gr_line (start 118.235886 113.778991) (end 119.37862 114.435926) (stroke (width 0.072) (type default)) (layer "Edge.Cuts"))
 (gr_line (start 94.696372 115.450622) (end 96.036094 114.254803) (stroke (width 0.072) (type default)) (layer "Edge.Cuts"))
 (gr_line (start 122.428003 107.902729) (end 124.833837 106.221273) (stroke (width 0.072) (type default)) (layer "Edge.Cuts"))
 (gr_line (start 96.915682 95.870046) (end 96.300723 95.934968) (stroke (width 0.072) (type default)) (layer "Edge.Cuts"))
 (gr_line (start 101.267221 90.780067) (end 101.426539 91.165324) (stroke (width 0.072) (type default)) (layer "Edge.Cuts"))
 (gr_line (start 93.386307 101.668875) (end 89.466663 102.437306) (stroke (width 0.072) (type default)) (layer "Edge.Cuts"))
 (gr_line (start 89.785277 86.506532) (end 89.616617 86.624835) (stroke (width 0.072) (type default)) (layer "Edge.Cuts"))
 (gr_line (start 92.127333 105.259764) (end 93.115417 105.684808) (stroke (width 0.072) (type default)) (layer "Edge.Cuts"))
 (gr_line (start 117.810863 113.531919) (end 118.235886 113.778991) (stroke (width 0.072) (type default)) (layer "Edge.Cuts"))
 (gr_line (start 103.577079 90.698401) (end 100.667829 89.017593) (stroke (width 0.072) (type default)) (layer "Edge.Cuts"))
 (gr_line (start 95.415429 111.114087) (end 95.162698 111.895604) (stroke (width 0.072) (type default)) (layer "Edge.Cuts"))
 (gr_line (start 90.453192 104.447888) (end 92.127333 105.259764) (stroke (width 0.072) (type default)) (layer "Edge.Cuts"))
 (gr_line (start 97.387966 113.079648) (end 96.101999 116.329238) (stroke (width 0.072) (type default)) (layer "Edge.Cuts"))
 (gr_line (start 101.145257 90.971115) (end 92.565917 87.396459) (stroke (width 0.072) (type default)) (layer "Edge.Cuts"))
 (gr_line (start 95.145569 111.187344) (end 95.415429 111.114087) (stroke (width 0.072) (type default)) (layer "Edge.Cuts"))
 (gr_line (start 120.074075 114.16949) (end 120.930868 114.5893) (stroke (width 0.072) (type default)) (layer "Edge.Cuts"))
 (gr_line (start 95.915177 116.759514) (end 97.315311 116.614005) (stroke (width 0.072) (type default)) (layer "Edge.Cuts"))
 (gr_line (start 92.987751 100.319415) (end 94.206253 101.349577) (stroke (width 0.072) (type default)) (layer "Edge.Cuts"))
 (gr_line (start 94.206253 101.349577) (end 93.386307 101.668875) (stroke (width 0.072) (type default)) (layer "Edge.Cuts"))
 (gr_line (start 115.18188 96.405078) (end 114.051603 95.15299) (stroke (width 0.072) (type default)) (layer "Edge.Cuts"))
 (gr_line (start 117.080207 99.295068) (end 116.830075 99.051135) (stroke (width 0.072) (type default)) (layer "Edge.Cuts"))
 (gr_line (start 107.648247 92.777552) (end 103.577079 90.698401) (stroke (width 0.072) (type default)) (layer "Edge.Cuts"))
 (gr_line (start 100.068875 115.075578) (end 100.664632 114.606562) (stroke (width 0.072) (type default)) (layer "Edge.Cuts"))
 (gr_line (start 112.126243 109.857306) (end 112.843954 110.54983) (stroke (width 0.072) (type default)) (layer "Edge.Cuts"))
 (gr_line (start 111.444335 109.920093) (end 112.126243 109.857306) (stroke (width 0.072) (type default)) (layer "Edge.Cuts"))
 (gr_line (start 119.37862 114.435926) (end 119.454414 114.089401) (stroke (width 0.072) (type default)) (layer "Edge.Cuts"))
 (gr_line (start 100.667829 89.017593) (end 100.81158 89.839941) (stroke (width 0.072) (type default)) (layer "Edge.Cuts"))
 (gr_line (start 89.616617 86.624835) (end 96.488585 95.403651) (stroke (width 0.072) (type default)) (layer "Edge.Cuts"))
 (gr_line (start 116.812918 113.532459) (end 117.565109 113.815542) (stroke (width 0.072) (type default)) (layer "Edge.Cuts"))
 (gr_line (start 101.749751 115.449837) (end 103.783121 112.931871) (stroke (width 0.072) (type default)) (layer "Edge.Cuts"))
 (gr_line (start 88.892679 95.341371) (end 88.607541 95.628889) (stroke (width 0.072) (type default)) (layer "Edge.Cuts"))
 (gr_line (start 100.81158 89.839941) (end 101.267221 90.780067) (stroke (width 0.072) (type default)) (layer "Edge.Cuts"))
 (gr_line (start 89.357017 96.751333) (end 92.987751 100.319415) (stroke (width 0.072) (type default)) (layer "Edge.Cuts"))
 (gr_line (start 92.69299 106.321332) (end 90.529206 108.860581) (stroke (width 0.072) (type default)) (layer "Edge.Cuts"))
 (gr_line (start 87.838188 102.607953) (end 90.453192 104.447888) (stroke (width 0.072) (type default)) (layer "Edge.Cuts"))
 (gr_line (start 119.597651 100.176042) (end 118.311173 99.793912) (stroke (width 0.072) (type default)) (layer "Edge.Cuts"))
 (gr_line (start 121.014888 113.038305) (end 121.366741 109.244337) (stroke (width 0.072) (type default)) (layer "Edge.Cuts"))
 (segment (start 100.095 106.195) (end 100.095 109.7925) (width 0.2) (layer "B.Cu") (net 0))
 (segment (start 101.365 100.270001) (end 101.004999 99.91) (width 0.2) (layer "B.Cu") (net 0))
 (segment (start 101.739744 111.47) (end 102.635 110.574744) (width 0.2) (layer "B.Cu") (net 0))
 (segment (start 102.635 106.195) (end 102.635 105.220001) (width 0.2) (layer "B.Cu") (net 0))
 (segment (start 107.08 106.465) (end 110.89 106.465) (width 0.2) (layer "B.Cu") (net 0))
 (segment (start 100.095 105.400552) (end 103.905 101.590552) (width 0.2) (layer "B.Cu") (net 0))
 (segment (start 105.535 104.92) (end 107.08 106.465) (width 0.2) (layer "B.Cu") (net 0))
 (segment (start 102.935001 104.92) (end 105.535 104.92) (width 0.2) (layer "B.Cu") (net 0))
 (segment (start 103.905 101.245) (end 115.146 101.245) (width 0.2) (layer "B.Cu") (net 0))
 (segment (start 115.146 101.245) (end 117.24 103.339) (width 0.2) (layer "B.Cu") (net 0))
 (segment (start 111.0125 97.48) (end 104.43 97.48) (width 0.2) (layer "B.Cu") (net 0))
 (segment (start 95.65 109.365686) (end 97.754314 111.47) (width 0.2) (layer "B.Cu") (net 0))
 (segment (start 100.095 109.7925) (end 99.8175 110.07) (width 0.2) (layer "B.Cu") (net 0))
 (segment (start 102.635 105.220001) (end 102.935001 104.92) (width 0.2) (layer "B.Cu") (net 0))
 (segment (start 111.8675 99.6175) (end 112.16 99.91) (width 0.2) (layer "B.Cu") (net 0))
 (segment (start 101.365 106.195) (end 101.365 109.7925) (width 0.2) (layer "B.Cu") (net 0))
 (segment (start 101.004999 99.91) (end 99.2675 99.91) (width 0.2) (layer "B.Cu") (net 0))
 (segment (start 101.365 101.245) (end 101.365 100.270001) (width 0.2) (layer "B.Cu") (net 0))
 (segment (start 102.635 110.574744) (end 102.635 106.195) (width 0.2) (layer "B.Cu") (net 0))
 (segment (start 99.2675 99.91) (end 96.92 102.2575) (width 0.2) (layer "B.Cu") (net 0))
 (segment (start 96.92 102.2575) (end 95.65 103.5275) (width 0.2) (layer "B.Cu") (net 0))
 (segment (start 104.43 97.48) (end 102.635 99.275) (width 0.2) (layer "B.Cu") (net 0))
 (segment (start 95.65 103.5275) (end 95.65 109.365686) (width 0.2) (layer "B.Cu") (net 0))
 (segment (start 96.92 110.07) (end 97.92 111.07) (width 0.2) (layer "B.Cu") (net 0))
 (segment (start 112.8875 99.1825) (end 112.16 99.91) (width 0.2) (layer "B.Cu") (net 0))
 (segment (start 100.095 106.195) (end 100.095 105.400552) (width 0.2) (layer "B.Cu") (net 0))
 (segment (start 97.754314 111.47) (end 101.739744 111.47) (width 0.2) (layer "B.Cu") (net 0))
 (segment (start 102.635 99.275) (end 102.635 101.245) (width 0.2) (layer "B.Cu") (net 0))
 (segment (start 101.365 109.7925) (end 101.6425 110.07) (width 0.2) (layer "B.Cu") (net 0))
 (segment (start 103.905 101.590552) (end 103.905 101.245) (width 0.2) (layer "B.Cu") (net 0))
 (segment (start 100.6425 111.07) (end 101.6425 110.07) (width 0.2) (layer "B.Cu") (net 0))
 (segment (start 96.92 105.1825) (end 96.92 110.07) (width 0.2) (layer "B.Cu") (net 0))
 (segment (start 112.8875 97.48) (end 112.8875 99.1825) (width 0.2) (layer "B.Cu") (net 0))
 (segment (start 97.92 111.07) (end 100.6425 111.07) (width 0.2) (layer "B.Cu") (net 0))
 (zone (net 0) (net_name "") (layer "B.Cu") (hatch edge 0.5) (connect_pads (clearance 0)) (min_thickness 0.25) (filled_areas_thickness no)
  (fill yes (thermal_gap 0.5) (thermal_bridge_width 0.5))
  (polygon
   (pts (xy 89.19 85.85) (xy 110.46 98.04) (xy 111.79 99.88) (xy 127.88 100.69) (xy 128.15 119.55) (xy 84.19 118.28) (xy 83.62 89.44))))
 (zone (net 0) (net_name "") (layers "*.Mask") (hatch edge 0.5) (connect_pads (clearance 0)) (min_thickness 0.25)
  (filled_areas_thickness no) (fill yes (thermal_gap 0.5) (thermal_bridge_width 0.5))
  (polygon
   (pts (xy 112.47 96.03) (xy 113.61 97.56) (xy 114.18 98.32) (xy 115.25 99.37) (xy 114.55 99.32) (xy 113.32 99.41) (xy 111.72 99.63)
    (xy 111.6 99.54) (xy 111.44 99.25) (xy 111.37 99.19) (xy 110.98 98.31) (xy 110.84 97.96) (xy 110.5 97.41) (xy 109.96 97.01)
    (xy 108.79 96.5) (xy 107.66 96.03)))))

